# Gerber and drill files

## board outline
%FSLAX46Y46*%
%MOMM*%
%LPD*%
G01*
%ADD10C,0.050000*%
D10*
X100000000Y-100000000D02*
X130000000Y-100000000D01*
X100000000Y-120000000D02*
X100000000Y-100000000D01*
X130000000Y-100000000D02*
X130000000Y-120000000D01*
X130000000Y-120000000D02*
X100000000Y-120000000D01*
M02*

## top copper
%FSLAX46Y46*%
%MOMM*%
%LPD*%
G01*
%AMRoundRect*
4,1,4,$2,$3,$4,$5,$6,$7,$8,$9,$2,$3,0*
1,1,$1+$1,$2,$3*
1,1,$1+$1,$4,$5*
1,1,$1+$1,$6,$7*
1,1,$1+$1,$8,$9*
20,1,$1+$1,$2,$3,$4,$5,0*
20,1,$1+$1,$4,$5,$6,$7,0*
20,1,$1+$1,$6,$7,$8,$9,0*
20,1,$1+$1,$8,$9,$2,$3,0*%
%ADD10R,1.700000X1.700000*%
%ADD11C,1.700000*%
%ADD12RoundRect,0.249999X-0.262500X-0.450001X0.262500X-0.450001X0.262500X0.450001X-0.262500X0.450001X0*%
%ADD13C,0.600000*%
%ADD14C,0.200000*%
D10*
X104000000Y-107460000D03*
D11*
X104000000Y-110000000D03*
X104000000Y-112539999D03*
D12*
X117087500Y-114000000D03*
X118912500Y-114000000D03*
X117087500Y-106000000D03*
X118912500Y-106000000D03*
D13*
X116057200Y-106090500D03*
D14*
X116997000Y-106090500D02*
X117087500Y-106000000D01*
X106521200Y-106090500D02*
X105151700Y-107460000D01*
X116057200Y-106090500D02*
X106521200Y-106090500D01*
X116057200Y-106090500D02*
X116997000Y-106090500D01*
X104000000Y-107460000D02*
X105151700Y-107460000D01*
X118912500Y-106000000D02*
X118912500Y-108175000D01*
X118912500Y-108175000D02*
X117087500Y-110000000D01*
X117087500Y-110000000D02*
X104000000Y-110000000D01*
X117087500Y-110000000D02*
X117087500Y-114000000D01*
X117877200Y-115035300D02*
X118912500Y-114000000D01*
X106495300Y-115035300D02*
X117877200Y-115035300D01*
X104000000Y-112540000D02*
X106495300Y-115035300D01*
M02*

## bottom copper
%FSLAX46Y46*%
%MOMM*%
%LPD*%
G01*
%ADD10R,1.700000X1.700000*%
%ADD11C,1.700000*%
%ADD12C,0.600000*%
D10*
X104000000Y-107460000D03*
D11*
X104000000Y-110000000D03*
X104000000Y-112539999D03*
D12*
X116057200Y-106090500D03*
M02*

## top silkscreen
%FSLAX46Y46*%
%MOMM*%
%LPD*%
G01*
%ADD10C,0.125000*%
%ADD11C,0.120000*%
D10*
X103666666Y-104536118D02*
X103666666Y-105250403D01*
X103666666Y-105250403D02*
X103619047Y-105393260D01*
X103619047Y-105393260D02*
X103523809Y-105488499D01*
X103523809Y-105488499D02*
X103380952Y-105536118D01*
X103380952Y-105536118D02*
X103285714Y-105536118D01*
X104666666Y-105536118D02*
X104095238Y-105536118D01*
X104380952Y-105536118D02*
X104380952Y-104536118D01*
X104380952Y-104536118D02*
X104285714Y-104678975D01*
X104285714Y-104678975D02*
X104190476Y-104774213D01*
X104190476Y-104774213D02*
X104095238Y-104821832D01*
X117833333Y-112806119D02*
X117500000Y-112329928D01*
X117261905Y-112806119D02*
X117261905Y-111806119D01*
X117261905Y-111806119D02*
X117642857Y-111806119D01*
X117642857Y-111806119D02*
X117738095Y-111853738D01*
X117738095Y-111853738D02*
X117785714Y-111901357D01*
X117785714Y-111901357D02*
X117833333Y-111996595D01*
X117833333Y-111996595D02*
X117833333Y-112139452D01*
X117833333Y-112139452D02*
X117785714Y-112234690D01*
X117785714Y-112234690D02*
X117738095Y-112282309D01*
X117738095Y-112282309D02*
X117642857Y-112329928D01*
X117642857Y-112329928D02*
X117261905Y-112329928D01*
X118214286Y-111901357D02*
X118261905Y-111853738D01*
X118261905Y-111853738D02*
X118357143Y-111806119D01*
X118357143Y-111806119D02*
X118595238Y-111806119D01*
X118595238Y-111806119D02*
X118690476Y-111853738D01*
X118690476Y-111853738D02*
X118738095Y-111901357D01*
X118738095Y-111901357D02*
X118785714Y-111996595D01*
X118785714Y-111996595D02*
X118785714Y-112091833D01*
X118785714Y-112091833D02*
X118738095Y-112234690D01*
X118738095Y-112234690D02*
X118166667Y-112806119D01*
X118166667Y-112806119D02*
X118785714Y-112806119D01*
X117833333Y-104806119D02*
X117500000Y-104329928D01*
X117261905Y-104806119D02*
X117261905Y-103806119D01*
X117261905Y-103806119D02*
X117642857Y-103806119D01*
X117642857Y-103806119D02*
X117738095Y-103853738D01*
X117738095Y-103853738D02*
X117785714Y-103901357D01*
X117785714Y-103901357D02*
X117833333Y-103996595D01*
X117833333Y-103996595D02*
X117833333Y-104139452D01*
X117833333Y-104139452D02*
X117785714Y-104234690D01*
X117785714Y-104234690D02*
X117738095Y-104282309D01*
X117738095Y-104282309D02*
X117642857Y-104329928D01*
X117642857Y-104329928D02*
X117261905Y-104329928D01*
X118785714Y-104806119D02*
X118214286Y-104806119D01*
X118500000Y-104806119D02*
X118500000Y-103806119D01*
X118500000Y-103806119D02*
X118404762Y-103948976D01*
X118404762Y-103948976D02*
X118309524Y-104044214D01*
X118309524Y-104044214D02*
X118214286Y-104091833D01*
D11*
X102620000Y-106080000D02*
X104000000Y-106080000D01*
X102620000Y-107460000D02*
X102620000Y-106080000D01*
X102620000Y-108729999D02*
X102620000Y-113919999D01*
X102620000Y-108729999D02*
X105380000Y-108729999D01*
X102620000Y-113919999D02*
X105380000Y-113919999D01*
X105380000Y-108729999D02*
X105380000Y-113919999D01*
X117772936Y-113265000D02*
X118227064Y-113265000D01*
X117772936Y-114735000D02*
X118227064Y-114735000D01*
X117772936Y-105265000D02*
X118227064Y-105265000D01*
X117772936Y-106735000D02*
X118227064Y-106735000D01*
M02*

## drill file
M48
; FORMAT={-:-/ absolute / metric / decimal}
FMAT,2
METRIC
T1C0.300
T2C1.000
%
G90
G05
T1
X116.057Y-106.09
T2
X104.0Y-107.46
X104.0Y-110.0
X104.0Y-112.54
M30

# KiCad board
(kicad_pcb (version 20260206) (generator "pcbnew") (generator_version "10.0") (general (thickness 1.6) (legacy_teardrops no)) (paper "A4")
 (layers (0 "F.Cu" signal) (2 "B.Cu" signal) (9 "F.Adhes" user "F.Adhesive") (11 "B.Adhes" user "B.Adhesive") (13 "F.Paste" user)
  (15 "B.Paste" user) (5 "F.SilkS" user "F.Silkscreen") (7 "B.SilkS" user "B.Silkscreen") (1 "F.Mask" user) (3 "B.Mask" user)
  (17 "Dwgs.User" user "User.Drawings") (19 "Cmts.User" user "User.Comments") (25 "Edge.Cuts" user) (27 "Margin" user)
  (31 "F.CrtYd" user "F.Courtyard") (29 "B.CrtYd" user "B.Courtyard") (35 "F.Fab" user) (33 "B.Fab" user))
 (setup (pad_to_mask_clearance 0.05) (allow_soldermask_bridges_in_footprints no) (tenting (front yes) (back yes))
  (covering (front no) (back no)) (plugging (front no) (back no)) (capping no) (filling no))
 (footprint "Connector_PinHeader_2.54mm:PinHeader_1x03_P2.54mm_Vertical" (layer "F.Cu") (at 104 107.46)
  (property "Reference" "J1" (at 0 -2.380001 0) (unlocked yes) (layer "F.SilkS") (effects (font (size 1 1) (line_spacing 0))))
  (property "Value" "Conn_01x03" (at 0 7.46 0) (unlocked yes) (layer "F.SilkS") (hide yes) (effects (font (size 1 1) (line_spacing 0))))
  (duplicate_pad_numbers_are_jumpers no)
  (fp_line (start -1.38 -1.38) (end 0 -1.38) (stroke (width 0.12) (type default)) (layer "F.SilkS"))
  (fp_line (start -1.38 0) (end -1.38 -1.38) (stroke (width 0.12) (type default)) (layer "F.SilkS"))
  (fp_line (start -1.38 1.269999) (end -1.38 6.459999) (stroke (width 0.12) (type default)) (layer "F.SilkS"))
  (fp_line (start -1.38 1.269999) (end 1.38 1.269999) (stroke (width 0.12) (type default)) (layer "F.SilkS"))
  (fp_line (start -1.38 6.459999) (end 1.38 6.459999) (stroke (width 0.12) (type default)) (layer "F.SilkS"))
  (fp_line (start 1.38 1.269999) (end 1.38 6.459999) (stroke (width 0.12) (type default)) (layer "F.SilkS"))
  (pad "1" thru_hole rect (at 0 0) (size 1.7 1.7) (drill 1) (layers "*.Cu" "*.Mask") (remove_unused_layers no) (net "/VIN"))
  (pad "2" thru_hole circle (at 0 2.54) (size 1.7 1.7) (drill 1) (layers "*.Cu" "*.Mask") (remove_unused_layers no) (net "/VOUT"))
  (pad "3" thru_hole circle (at 0 5.079999) (size 1.7 1.7) (drill 1) (layers "*.Cu" "*.Mask") (remove_unused_layers no) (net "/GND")))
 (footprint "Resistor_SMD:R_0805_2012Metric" (layer "F.Cu") (at 118 114)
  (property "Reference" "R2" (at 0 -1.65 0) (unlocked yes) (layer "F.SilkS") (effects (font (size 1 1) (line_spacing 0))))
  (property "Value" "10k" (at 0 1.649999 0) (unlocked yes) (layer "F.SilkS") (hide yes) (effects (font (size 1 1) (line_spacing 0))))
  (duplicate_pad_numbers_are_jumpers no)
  (fp_line (start -0.227064 -0.735) (end 0.227064 -0.735) (stroke (width 0.12) (type default)) (layer "F.SilkS"))
  (fp_line (start -0.227064 0.735) (end 0.227064 0.735) (stroke (width 0.12) (type default)) (layer "F.SilkS"))
  (pad "1" smd roundrect (at -0.9125 0) (size 1.024999 1.4) (layers "F.Cu" "F.Mask" "F.Paste") (roundrect_rratio 0.243902) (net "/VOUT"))
  (pad "2" smd roundrect (at 0.9125 0) (size 1.024999 1.4) (layers "F.Cu" "F.Mask" "F.Paste") (roundrect_rratio 0.243902) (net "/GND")))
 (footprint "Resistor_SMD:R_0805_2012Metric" (layer "F.Cu") (at 118 106)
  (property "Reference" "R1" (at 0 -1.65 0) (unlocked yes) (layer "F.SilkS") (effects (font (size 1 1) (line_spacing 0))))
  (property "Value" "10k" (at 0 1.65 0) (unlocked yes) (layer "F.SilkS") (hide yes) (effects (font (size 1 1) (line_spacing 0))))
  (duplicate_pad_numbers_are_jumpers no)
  (fp_line (start -0.227064 -0.735) (end 0.227064 -0.735) (stroke (width 0.12) (type default)) (layer "F.SilkS"))
  (fp_line (start -0.227064 0.735) (end 0.227064 0.735) (stroke (width 0.12) (type default)) (layer "F.SilkS"))
  (pad "1" smd roundrect (at -0.9125 0) (size 1.024999 1.4) (layers "F.Cu" "F.Mask" "F.Paste") (roundrect_rratio 0.243902) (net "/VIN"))
  (pad "2" smd roundrect (at 0.9125 0) (size 1.024999 1.4) (layers "F.Cu" "F.Mask" "F.Paste") (roundrect_rratio 0.243902) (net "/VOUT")))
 (gr_line (start 100 100) (end 130 100) (stroke (width 0.05) (type default)) (layer "Edge.Cuts"))
 (gr_line (start 100 120) (end 100 100) (stroke (width 0.05) (type default)) (layer "Edge.Cuts"))
 (gr_line (start 130 100) (end 130 120) (stroke (width 0.05) (type default)) (layer "Edge.Cuts"))
 (gr_line (start 130 120) (end 100 120) (stroke (width 0.05) (type default)) (layer "Edge.Cuts"))
 (segment (start 116.997 106.0905) (end 117.0875 106) (width 0.2) (layer "F.Cu") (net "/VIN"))
 (segment (start 106.5212 106.0905) (end 105.1517 107.46) (width 0.2) (layer "F.Cu") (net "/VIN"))
 (segment (start 116.0572 106.0905) (end 106.5212 106.0905) (width 0.2) (layer "F.Cu") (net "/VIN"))
 (segment (start 116.0572 106.0905) (end 116.997 106.0905) (width 0.2) (layer "F.Cu") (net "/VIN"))
 (segment (start 104 107.46) (end 105.1517 107.46) (width 0.2) (layer "F.Cu") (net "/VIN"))
 (via (at 116.0572 106.0905) (size 0.6) (drill 0.3) (layers "F.Cu" "B.Cu") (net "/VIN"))
 (segment (start 118.9125 106) (end 118.9125 108.175) (width 0.2) (layer "F.Cu") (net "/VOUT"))
 (segment (start 118.9125 108.175) (end 117.0875 110) (width 0.2) (layer "F.Cu") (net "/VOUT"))
 (segment (start 117.0875 110) (end 104 110) (width 0.2) (layer "F.Cu") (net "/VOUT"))
 (segment (start 117.0875 110) (end 117.0875 114) (width 0.2) (layer "F.Cu") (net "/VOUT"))
 (segment (start 117.8772 115.0353) (end 118.9125 114) (width 0.2) (layer "F.Cu") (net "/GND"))
 (segment (start 106.4953 115.0353) (end 117.8772 115.0353) (width 0.2) (layer "F.Cu") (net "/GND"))
 (segment (start 104 112.54) (end 106.4953 115.0353) (width 0.2) (layer "F.Cu") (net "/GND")))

